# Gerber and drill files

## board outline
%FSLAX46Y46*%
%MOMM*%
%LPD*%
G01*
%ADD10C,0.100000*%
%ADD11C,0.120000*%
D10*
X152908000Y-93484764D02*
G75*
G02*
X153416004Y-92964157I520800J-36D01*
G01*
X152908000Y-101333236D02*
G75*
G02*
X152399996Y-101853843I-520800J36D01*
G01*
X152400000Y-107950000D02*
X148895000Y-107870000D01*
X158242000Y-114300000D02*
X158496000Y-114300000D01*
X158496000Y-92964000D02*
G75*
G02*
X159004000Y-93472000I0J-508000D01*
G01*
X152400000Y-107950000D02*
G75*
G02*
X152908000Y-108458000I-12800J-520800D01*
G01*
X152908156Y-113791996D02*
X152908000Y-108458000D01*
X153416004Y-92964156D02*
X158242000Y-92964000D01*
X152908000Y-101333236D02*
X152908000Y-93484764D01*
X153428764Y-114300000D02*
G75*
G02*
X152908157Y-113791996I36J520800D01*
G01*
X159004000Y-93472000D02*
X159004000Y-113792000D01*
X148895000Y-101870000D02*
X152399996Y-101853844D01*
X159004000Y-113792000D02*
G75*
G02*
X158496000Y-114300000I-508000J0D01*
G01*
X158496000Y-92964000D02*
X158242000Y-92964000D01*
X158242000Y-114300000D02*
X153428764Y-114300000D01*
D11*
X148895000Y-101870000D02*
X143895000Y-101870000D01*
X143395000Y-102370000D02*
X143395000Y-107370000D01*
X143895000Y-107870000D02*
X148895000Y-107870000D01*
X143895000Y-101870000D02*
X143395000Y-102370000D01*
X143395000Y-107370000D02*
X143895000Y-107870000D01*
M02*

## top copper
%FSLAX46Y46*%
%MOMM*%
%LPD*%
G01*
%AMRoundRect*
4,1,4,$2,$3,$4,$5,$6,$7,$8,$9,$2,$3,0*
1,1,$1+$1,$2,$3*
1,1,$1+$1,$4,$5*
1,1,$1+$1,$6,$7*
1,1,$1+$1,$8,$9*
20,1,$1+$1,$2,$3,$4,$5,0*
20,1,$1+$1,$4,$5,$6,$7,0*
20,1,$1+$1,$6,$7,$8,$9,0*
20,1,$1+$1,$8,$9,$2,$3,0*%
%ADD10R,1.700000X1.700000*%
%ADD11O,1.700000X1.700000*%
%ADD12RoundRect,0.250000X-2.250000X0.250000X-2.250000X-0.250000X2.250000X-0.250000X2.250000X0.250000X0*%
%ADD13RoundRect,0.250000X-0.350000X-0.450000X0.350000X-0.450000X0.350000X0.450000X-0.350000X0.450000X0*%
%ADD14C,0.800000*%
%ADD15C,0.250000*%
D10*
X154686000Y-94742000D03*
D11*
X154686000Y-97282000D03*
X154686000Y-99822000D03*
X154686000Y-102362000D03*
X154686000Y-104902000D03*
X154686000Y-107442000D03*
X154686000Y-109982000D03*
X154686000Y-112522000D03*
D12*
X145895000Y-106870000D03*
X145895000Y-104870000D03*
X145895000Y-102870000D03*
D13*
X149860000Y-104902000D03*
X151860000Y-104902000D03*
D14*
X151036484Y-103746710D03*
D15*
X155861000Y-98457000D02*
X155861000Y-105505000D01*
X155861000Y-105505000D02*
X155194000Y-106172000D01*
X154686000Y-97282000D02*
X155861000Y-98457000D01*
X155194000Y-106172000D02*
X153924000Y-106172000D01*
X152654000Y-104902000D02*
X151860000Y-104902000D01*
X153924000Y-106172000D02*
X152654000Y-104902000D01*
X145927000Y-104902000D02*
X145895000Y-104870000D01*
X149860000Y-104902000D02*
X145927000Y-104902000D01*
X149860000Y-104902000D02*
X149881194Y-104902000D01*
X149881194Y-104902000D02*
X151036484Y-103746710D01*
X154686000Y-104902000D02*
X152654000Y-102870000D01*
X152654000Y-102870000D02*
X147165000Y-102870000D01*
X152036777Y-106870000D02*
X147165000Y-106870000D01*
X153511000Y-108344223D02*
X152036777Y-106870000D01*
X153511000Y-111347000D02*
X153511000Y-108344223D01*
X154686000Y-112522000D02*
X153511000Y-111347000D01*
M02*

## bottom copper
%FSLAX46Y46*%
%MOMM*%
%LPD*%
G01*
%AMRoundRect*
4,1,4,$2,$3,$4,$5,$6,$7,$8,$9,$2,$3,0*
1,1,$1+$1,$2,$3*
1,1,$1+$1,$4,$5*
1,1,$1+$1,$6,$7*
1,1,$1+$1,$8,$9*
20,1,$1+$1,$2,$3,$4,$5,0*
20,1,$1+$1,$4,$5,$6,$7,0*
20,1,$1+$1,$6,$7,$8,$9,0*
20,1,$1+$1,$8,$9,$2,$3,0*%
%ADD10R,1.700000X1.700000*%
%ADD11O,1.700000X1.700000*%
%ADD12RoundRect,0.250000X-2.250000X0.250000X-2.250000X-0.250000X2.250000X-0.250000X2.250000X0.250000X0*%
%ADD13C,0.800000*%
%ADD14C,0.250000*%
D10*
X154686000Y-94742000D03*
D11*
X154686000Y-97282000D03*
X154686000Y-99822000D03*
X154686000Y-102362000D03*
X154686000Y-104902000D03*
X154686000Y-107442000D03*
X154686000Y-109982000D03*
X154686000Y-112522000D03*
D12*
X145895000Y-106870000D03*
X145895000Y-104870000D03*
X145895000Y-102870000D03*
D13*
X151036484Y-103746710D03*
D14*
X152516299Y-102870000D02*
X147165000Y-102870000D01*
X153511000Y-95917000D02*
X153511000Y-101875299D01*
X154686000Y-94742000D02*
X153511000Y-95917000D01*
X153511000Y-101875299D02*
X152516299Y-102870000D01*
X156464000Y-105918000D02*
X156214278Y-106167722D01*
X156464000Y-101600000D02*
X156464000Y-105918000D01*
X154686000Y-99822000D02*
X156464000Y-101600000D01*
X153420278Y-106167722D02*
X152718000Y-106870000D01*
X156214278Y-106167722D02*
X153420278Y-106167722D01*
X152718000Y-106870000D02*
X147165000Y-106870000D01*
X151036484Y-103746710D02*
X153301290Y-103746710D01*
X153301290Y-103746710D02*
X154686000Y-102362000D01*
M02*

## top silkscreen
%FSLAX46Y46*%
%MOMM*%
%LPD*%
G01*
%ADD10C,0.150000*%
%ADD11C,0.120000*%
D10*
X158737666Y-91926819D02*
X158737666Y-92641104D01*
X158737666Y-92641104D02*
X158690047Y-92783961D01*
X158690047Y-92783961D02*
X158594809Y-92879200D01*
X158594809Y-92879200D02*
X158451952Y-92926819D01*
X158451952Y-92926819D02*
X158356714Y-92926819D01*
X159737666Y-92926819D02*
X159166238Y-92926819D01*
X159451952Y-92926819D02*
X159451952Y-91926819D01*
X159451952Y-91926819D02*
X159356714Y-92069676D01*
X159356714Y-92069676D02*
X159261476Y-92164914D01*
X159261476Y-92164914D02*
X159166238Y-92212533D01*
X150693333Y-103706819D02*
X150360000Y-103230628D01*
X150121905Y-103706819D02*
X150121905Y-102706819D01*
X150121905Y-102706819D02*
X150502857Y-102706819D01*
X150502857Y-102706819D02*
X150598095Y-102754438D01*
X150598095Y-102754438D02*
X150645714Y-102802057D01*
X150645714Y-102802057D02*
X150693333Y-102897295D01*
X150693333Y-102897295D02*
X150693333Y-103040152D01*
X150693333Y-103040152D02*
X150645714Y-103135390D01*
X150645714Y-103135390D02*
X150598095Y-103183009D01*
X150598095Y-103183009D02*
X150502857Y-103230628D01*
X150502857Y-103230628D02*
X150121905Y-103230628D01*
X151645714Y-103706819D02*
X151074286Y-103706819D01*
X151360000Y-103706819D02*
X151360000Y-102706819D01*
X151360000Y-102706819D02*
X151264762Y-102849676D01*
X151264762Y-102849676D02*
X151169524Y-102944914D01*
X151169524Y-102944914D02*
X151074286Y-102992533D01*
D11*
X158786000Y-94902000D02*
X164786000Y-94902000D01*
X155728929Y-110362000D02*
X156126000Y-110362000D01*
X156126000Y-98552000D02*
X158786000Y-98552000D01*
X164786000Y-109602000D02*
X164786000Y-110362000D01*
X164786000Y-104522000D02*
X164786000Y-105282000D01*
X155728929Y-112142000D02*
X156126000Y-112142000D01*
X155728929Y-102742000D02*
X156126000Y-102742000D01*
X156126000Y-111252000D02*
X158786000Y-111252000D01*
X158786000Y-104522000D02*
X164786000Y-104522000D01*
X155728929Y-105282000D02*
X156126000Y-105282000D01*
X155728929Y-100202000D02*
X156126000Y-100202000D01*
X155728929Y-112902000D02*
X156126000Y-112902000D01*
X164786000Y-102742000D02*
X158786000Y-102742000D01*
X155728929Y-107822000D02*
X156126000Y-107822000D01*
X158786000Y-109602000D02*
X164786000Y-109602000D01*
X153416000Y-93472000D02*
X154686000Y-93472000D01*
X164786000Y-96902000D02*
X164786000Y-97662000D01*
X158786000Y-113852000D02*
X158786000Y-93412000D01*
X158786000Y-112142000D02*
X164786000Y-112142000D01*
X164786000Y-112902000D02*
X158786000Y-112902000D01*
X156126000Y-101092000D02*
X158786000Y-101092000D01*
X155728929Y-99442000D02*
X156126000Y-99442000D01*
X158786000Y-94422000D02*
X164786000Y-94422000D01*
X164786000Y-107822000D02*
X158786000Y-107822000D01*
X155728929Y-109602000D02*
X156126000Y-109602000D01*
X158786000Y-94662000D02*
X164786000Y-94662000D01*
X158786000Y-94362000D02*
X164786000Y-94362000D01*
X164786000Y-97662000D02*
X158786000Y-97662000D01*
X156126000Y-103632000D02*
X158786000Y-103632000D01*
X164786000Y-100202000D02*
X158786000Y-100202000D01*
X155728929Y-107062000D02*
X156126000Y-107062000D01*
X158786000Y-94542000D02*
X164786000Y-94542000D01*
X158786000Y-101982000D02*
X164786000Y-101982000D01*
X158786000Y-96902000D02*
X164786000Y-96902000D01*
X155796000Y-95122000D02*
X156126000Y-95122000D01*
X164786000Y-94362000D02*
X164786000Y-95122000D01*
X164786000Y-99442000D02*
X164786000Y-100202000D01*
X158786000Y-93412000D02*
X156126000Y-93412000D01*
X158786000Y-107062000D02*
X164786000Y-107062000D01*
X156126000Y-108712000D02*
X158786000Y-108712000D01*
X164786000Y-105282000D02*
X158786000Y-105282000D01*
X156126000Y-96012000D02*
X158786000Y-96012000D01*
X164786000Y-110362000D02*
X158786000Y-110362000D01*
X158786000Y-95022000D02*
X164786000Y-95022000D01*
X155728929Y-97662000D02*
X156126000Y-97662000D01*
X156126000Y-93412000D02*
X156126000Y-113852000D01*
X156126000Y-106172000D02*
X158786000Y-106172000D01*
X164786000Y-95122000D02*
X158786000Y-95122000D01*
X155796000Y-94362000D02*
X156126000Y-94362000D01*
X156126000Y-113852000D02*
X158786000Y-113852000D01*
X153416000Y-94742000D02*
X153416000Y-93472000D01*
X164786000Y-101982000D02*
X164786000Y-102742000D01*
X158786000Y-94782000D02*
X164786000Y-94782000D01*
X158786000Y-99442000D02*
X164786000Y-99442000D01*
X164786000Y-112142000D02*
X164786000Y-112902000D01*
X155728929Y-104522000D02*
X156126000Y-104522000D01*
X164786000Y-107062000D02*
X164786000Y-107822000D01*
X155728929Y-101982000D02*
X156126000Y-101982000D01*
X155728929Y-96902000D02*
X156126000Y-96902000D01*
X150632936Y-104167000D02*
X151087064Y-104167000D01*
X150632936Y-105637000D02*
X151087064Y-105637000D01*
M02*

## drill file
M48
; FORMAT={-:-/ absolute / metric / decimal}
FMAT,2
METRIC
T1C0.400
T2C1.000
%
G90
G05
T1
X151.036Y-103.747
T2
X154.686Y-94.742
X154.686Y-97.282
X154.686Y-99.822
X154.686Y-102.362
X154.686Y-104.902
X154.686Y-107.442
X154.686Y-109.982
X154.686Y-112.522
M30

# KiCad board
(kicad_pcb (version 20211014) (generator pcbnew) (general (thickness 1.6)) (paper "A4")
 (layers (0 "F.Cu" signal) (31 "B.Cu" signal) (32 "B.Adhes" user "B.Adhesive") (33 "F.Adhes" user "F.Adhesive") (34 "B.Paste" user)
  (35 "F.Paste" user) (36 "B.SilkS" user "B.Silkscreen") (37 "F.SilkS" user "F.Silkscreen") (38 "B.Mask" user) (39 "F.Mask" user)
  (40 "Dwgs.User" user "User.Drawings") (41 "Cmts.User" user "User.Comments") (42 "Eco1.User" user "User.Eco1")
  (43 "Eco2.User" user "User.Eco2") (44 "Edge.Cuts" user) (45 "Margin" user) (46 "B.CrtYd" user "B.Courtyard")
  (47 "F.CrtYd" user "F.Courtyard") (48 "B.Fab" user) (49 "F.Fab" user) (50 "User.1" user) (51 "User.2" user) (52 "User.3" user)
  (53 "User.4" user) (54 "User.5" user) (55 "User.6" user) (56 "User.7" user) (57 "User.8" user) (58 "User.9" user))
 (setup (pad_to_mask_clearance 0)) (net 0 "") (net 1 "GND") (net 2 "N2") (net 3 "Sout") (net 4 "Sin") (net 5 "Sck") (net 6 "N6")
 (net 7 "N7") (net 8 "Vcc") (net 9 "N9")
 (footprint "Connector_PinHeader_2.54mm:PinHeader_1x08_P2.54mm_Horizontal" (layer "F.Cu") (at 154.686 94.742)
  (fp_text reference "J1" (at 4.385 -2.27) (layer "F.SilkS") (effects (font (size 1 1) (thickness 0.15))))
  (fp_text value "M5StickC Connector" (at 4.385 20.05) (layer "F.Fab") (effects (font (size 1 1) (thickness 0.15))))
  (fp_line (start 4.1 0.16) (end 10.1 0.16) (layer "F.SilkS") (width 0.12))
  (fp_line (start 1.042929 15.62) (end 1.44 15.62) (layer "F.SilkS") (width 0.12))
  (fp_line (start 1.44 3.81) (end 4.1 3.81) (layer "F.SilkS") (width 0.12))
  (fp_line (start 10.1 14.86) (end 10.1 15.62) (layer "F.SilkS") (width 0.12))
  (fp_line (start 10.1 9.78) (end 10.1 10.54) (layer "F.SilkS") (width 0.12))
  (fp_line (start 1.042929 17.4) (end 1.44 17.4) (layer "F.SilkS") (width 0.12))
  (fp_line (start 1.042929 8) (end 1.44 8) (layer "F.SilkS") (width 0.12))
  (fp_line (start 1.44 16.51) (end 4.1 16.51) (layer "F.SilkS") (width 0.12))
  (fp_line (start 4.1 9.78) (end 10.1 9.78) (layer "F.SilkS") (width 0.12))
  (fp_line (start 1.042929 10.54) (end 1.44 10.54) (layer "F.SilkS") (width 0.12))
  (fp_line (start 1.042929 5.46) (end 1.44 5.46) (layer "F.SilkS") (width 0.12))
  (fp_line (start 1.042929 18.16) (end 1.44 18.16) (layer "F.SilkS") (width 0.12))
  (fp_line (start 10.1 8) (end 4.1 8) (layer "F.SilkS") (width 0.12))
  (fp_line (start 1.042929 13.08) (end 1.44 13.08) (layer "F.SilkS") (width 0.12))
  (fp_line (start 4.1 14.86) (end 10.1 14.86) (layer "F.SilkS") (width 0.12))
  (fp_line (start -1.27 -1.27) (end 0 -1.27) (layer "F.SilkS") (width 0.12))
  (fp_line (start 10.1 2.16) (end 10.1 2.92) (layer "F.SilkS") (width 0.12))
  (fp_line (start 4.1 19.11) (end 4.1 -1.33) (layer "F.SilkS") (width 0.12))
  (fp_line (start 4.1 17.4) (end 10.1 17.4) (layer "F.SilkS") (width 0.12))
  (fp_line (start 10.1 18.16) (end 4.1 18.16) (layer "F.SilkS") (width 0.12))
  (fp_line (start 1.44 6.35) (end 4.1 6.35) (layer "F.SilkS") (width 0.12))
  (fp_line (start 1.042929 4.7) (end 1.44 4.7) (layer "F.SilkS") (width 0.12))
  (fp_line (start 4.1 -0.32) (end 10.1 -0.32) (layer "F.SilkS") (width 0.12))
  (fp_line (start 10.1 13.08) (end 4.1 13.08) (layer "F.SilkS") (width 0.12))
  (fp_line (start 1.042929 14.86) (end 1.44 14.86) (layer "F.SilkS") (width 0.12))
  (fp_line (start 4.1 -0.08) (end 10.1 -0.08) (layer "F.SilkS") (width 0.12))
  (fp_line (start 4.1 -0.38) (end 10.1 -0.38) (layer "F.SilkS") (width 0.12))
  (fp_line (start 10.1 2.92) (end 4.1 2.92) (layer "F.SilkS") (width 0.12))
  (fp_line (start 1.44 8.89) (end 4.1 8.89) (layer "F.SilkS") (width 0.12))
  (fp_line (start 10.1 5.46) (end 4.1 5.46) (layer "F.SilkS") (width 0.12))
  (fp_line (start 1.042929 12.32) (end 1.44 12.32) (layer "F.SilkS") (width 0.12))
  (fp_line (start 4.1 -0.2) (end 10.1 -0.2) (layer "F.SilkS") (width 0.12))
  (fp_line (start 4.1 7.24) (end 10.1 7.24) (layer "F.SilkS") (width 0.12))
  (fp_line (start 4.1 2.16) (end 10.1 2.16) (layer "F.SilkS") (width 0.12))
  (fp_line (start 1.11 0.38) (end 1.44 0.38) (layer "F.SilkS") (width 0.12))
  (fp_line (start 10.1 -0.38) (end 10.1 0.38) (layer "F.SilkS") (width 0.12))
  (fp_line (start 10.1 4.7) (end 10.1 5.46) (layer "F.SilkS") (width 0.12))
  (fp_line (start 4.1 -1.33) (end 1.44 -1.33) (layer "F.SilkS") (width 0.12))
  (fp_line (start 4.1 12.32) (end 10.1 12.32) (layer "F.SilkS") (width 0.12))
  (fp_line (start 1.44 13.97) (end 4.1 13.97) (layer "F.SilkS") (width 0.12))
  (fp_line (start 10.1 10.54) (end 4.1 10.54) (layer "F.SilkS") (width 0.12))
  (fp_line (start 1.44 1.27) (end 4.1 1.27) (layer "F.SilkS") (width 0.12))
  (fp_line (start 10.1 15.62) (end 4.1 15.62) (layer "F.SilkS") (width 0.12))
  (fp_line (start 4.1 0.28) (end 10.1 0.28) (layer "F.SilkS") (width 0.12))
  (fp_line (start 1.042929 2.92) (end 1.44 2.92) (layer "F.SilkS") (width 0.12))
  (fp_line (start 1.44 -1.33) (end 1.44 19.11) (layer "F.SilkS") (width 0.12))
  (fp_line (start 1.44 11.43) (end 4.1 11.43) (layer "F.SilkS") (width 0.12))
  (fp_line (start 10.1 0.38) (end 4.1 0.38) (layer "F.SilkS") (width 0.12))
  (fp_line (start 1.11 -0.38) (end 1.44 -0.38) (layer "F.SilkS") (width 0.12))
  (fp_line (start 1.44 19.11) (end 4.1 19.11) (layer "F.SilkS") (width 0.12))
  (fp_line (start -1.27 0) (end -1.27 -1.27) (layer "F.SilkS") (width 0.12))
  (fp_line (start 10.1 7.24) (end 10.1 8) (layer "F.SilkS") (width 0.12))
  (fp_line (start 4.1 0.04) (end 10.1 0.04) (layer "F.SilkS") (width 0.12))
  (fp_line (start 4.1 4.7) (end 10.1 4.7) (layer "F.SilkS") (width 0.12))
  (fp_line (start 10.1 17.4) (end 10.1 18.16) (layer "F.SilkS") (width 0.12))
  (fp_line (start 1.042929 9.78) (end 1.44 9.78) (layer "F.SilkS") (width 0.12))
  (fp_line (start 10.1 12.32) (end 10.1 13.08) (layer "F.SilkS") (width 0.12))
  (fp_line (start 1.042929 7.24) (end 1.44 7.24) (layer "F.SilkS") (width 0.12))
  (fp_line (start 1.042929 2.16) (end 1.44 2.16) (layer "F.SilkS") (width 0.12))
  (pad "1" thru_hole rect (at 0 0) (size 1.7 1.7) (drill 1) (layers *.Cu *.Mask) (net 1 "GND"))
  (pad "2" thru_hole oval (at 0 2.54) (size 1.7 1.7) (drill 1) (layers *.Cu *.Mask) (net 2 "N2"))
  (pad "3" thru_hole oval (at 0 5.08) (size 1.7 1.7) (drill 1) (layers *.Cu *.Mask) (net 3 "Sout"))
  (pad "4" thru_hole oval (at 0 7.62) (size 1.7 1.7) (drill 1) (layers *.Cu *.Mask) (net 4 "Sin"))
  (pad "5" thru_hole oval (at 0 10.16) (size 1.7 1.7) (drill 1) (layers *.Cu *.Mask) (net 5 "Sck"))
  (pad "6" thru_hole oval (at 0 12.7) (size 1.7 1.7) (drill 1) (layers *.Cu *.Mask) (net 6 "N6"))
  (pad "7" thru_hole oval (at 0 15.24) (size 1.7 1.7) (drill 1) (layers *.Cu *.Mask) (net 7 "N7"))
  (pad "8" thru_hole oval (at 0 17.78) (size 1.7 1.7) (drill 1) (layers *.Cu *.Mask) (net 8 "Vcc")))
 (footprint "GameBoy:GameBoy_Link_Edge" (layer "F.Cu") (at 143.395 102.37 -90)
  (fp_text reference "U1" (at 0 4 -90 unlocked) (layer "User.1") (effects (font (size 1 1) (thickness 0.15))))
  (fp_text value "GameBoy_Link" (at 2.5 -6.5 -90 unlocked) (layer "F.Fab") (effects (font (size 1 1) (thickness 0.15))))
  (fp_line (start -0.5 -5.5) (end -0.5 -0.5) (layer "Edge.Cuts") (width 0.12))
  (fp_line (start 0 0) (end 5 0) (layer "Edge.Cuts") (width 0.12))
  (fp_line (start 5.5 -0.5) (end 5.5 -5.5) (layer "Edge.Cuts") (width 0.12))
  (fp_line (start -0.5 -0.5) (end 0 0) (layer "Edge.Cuts") (width 0.12))
  (fp_line (start 5 0) (end 5.5 -0.5) (layer "Edge.Cuts") (width 0.12))
  (pad "1" smd roundrect (at 4.5 -2.5 270) (size 1 5) (layers "F.Cu" "F.Paste" "F.Mask") (roundrect_rratio 0.25) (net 8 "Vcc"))
  (pad "2" smd roundrect (at 4.5 -2.5 270) (size 1 5) (layers "B.Cu" "B.Paste" "B.Mask") (roundrect_rratio 0.25) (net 3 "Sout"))
  (pad "3" smd roundrect (at 2.5 -2.5 270) (size 1 5) (layers "F.Cu" "F.Paste" "F.Mask") (roundrect_rratio 0.25) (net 4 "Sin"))
  (pad "4" smd roundrect (at 2.5 -2.5 270) (size 1 5) (layers "B.Cu" "B.Paste" "B.Mask") (roundrect_rratio 0.25) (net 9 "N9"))
  (pad "5" smd roundrect (at 0.5 -2.5 270) (size 1 5) (layers "F.Cu" "F.Paste" "F.Mask") (roundrect_rratio 0.25) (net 5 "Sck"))
  (pad "6" smd roundrect (at 0.5 -2.5 270) (size 1 5) (layers "B.Cu" "B.Paste" "B.Mask") (roundrect_rratio 0.25) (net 1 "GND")))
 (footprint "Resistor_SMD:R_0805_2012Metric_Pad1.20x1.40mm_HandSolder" (layer "F.Cu") (at 150.86 104.902)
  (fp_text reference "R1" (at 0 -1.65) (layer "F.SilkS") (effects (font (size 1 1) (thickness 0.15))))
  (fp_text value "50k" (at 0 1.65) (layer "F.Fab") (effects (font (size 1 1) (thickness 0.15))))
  (fp_line (start -0.227064 -0.735) (end 0.227064 -0.735) (layer "F.SilkS") (width 0.12))
  (fp_line (start -0.227064 0.735) (end 0.227064 0.735) (layer "F.SilkS") (width 0.12))
  (pad "1" smd roundrect (at -1 0) (size 1.2 1.4) (layers "F.Cu" "F.Paste" "F.Mask") (roundrect_rratio 0.2083333333) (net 4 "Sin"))
  (pad "2" smd roundrect (at 1 0) (size 1.2 1.4) (layers "F.Cu" "F.Paste" "F.Mask") (roundrect_rratio 0.2083333333) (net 2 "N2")))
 (gr_arc (start 152.908 93.484764) (mid 153.056044 93.121068) (end 153.416004 92.964156) (layer "Edge.Cuts") (width 0.1))
 (gr_arc (start 152.908 101.333236) (mid 152.759956 101.696932) (end 152.399996 101.853844) (layer "Edge.Cuts") (width 0.1))
 (gr_line (start 152.4 107.95) (end 148.895 107.87) (layer "Edge.Cuts") (width 0.1))
 (gr_line (start 158.242 114.3) (end 158.496 114.3) (layer "Edge.Cuts") (width 0.1))
 (gr_arc (start 158.496 92.964) (mid 158.85521 93.11279) (end 159.004 93.472) (layer "Edge.Cuts") (width 0.1))
 (gr_arc (start 152.4 107.95) (mid 152.755582 108.102418) (end 152.908 108.458) (layer "Edge.Cuts") (width 0.1))
 (gr_line (start 152.908156 113.791996) (end 152.908 108.458) (layer "Edge.Cuts") (width 0.1))
 (gr_line (start 153.416004 92.964156) (end 158.242 92.964) (layer "Edge.Cuts") (width 0.1))
 (gr_line (start 152.908 101.333236) (end 152.908 93.484764) (layer "Edge.Cuts") (width 0.1))
 (gr_arc (start 153.428764 114.3) (mid 153.065068 114.151956) (end 152.908156 113.791996) (layer "Edge.Cuts") (width 0.1))
 (gr_line (start 159.004 93.472) (end 159.004 113.792) (layer "Edge.Cuts") (width 0.1))
 (gr_line (start 148.895 101.87) (end 152.399996 101.853844) (layer "Edge.Cuts") (width 0.1))
 (gr_arc (start 159.004 113.792) (mid 158.85521 114.15121) (end 158.496 114.3) (layer "Edge.Cuts") (width 0.1))
 (gr_line (start 158.496 92.964) (end 158.242 92.964) (layer "Edge.Cuts") (width 0.1))
 (gr_line (start 158.242 114.3) (end 153.428764 114.3) (layer "Edge.Cuts") (width 0.1))
 (segment (start 152.516299 102.87) (end 147.165 102.87) (width 0.25) (layer "B.Cu") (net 1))
 (segment (start 153.511 95.917) (end 153.511 101.875299) (width 0.25) (layer "B.Cu") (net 1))
 (segment (start 154.686 94.742) (end 153.511 95.917) (width 0.25) (layer "B.Cu") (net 1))
 (segment (start 153.511 101.875299) (end 152.516299 102.87) (width 0.25) (layer "B.Cu") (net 1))
 (segment (start 155.861 98.457) (end 155.861 105.505) (width 0.25) (layer "F.Cu") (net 2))
 (segment (start 155.861 105.505) (end 155.194 106.172) (width 0.25) (layer "F.Cu") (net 2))
 (segment (start 154.686 97.282) (end 155.861 98.457) (width 0.25) (layer "F.Cu") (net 2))
 (segment (start 155.194 106.172) (end 153.924 106.172) (width 0.25) (layer "F.Cu") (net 2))
 (segment (start 152.654 104.902) (end 151.86 104.902) (width 0.25) (layer "F.Cu") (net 2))
 (segment (start 153.924 106.172) (end 152.654 104.902) (width 0.25) (layer "F.Cu") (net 2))
 (segment (start 156.464 105.918) (end 156.214278 106.167722) (width 0.25) (layer "B.Cu") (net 3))
 (segment (start 156.464 101.6) (end 156.464 105.918) (width 0.25) (layer "B.Cu") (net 3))
 (segment (start 154.686 99.822) (end 156.464 101.6) (width 0.25) (layer "B.Cu") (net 3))
 (segment (start 153.420278 106.167722) (end 152.718 106.87) (width 0.25) (layer "B.Cu") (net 3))
 (segment (start 156.214278 106.167722) (end 153.420278 106.167722) (width 0.25) (layer "B.Cu") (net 3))
 (segment (start 152.718 106.87) (end 147.165 106.87) (width 0.25) (layer "B.Cu") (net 3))
 (segment (start 145.927 104.902) (end 145.895 104.87) (width 0.25) (layer "F.Cu") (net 4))
 (segment (start 149.86 104.902) (end 145.927 104.902) (width 0.25) (layer "F.Cu") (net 4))
 (segment (start 149.86 104.902) (end 149.881194 104.902) (width 0.25) (layer "F.Cu") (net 4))
 (segment (start 149.881194 104.902) (end 151.036484 103.74671) (width 0.25) (layer "F.Cu") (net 4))
 (via (at 151.036484 103.74671) (size 0.8) (drill 0.4) (layers "F.Cu" "B.Cu") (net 4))
 (segment (start 151.036484 103.74671) (end 153.30129 103.74671) (width 0.25) (layer "B.Cu") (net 4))
 (segment (start 153.30129 103.74671) (end 154.686 102.362) (width 0.25) (layer "B.Cu") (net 4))
 (segment (start 154.686 104.902) (end 152.654 102.87) (width 0.25) (layer "F.Cu") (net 5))
 (segment (start 152.654 102.87) (end 147.165 102.87) (width 0.25) (layer "F.Cu") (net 5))
 (segment (start 152.036777 106.87) (end 147.165 106.87) (width 0.25) (layer "F.Cu") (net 8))
 (segment (start 153.511 108.344223) (end 152.036777 106.87) (width 0.25) (layer "F.Cu") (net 8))
 (segment (start 153.511 111.347) (end 153.511 108.344223) (width 0.25) (layer "F.Cu") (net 8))
 (segment (start 154.686 112.522) (end 153.511 111.347) (width 0.25) (layer "F.Cu") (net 8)))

